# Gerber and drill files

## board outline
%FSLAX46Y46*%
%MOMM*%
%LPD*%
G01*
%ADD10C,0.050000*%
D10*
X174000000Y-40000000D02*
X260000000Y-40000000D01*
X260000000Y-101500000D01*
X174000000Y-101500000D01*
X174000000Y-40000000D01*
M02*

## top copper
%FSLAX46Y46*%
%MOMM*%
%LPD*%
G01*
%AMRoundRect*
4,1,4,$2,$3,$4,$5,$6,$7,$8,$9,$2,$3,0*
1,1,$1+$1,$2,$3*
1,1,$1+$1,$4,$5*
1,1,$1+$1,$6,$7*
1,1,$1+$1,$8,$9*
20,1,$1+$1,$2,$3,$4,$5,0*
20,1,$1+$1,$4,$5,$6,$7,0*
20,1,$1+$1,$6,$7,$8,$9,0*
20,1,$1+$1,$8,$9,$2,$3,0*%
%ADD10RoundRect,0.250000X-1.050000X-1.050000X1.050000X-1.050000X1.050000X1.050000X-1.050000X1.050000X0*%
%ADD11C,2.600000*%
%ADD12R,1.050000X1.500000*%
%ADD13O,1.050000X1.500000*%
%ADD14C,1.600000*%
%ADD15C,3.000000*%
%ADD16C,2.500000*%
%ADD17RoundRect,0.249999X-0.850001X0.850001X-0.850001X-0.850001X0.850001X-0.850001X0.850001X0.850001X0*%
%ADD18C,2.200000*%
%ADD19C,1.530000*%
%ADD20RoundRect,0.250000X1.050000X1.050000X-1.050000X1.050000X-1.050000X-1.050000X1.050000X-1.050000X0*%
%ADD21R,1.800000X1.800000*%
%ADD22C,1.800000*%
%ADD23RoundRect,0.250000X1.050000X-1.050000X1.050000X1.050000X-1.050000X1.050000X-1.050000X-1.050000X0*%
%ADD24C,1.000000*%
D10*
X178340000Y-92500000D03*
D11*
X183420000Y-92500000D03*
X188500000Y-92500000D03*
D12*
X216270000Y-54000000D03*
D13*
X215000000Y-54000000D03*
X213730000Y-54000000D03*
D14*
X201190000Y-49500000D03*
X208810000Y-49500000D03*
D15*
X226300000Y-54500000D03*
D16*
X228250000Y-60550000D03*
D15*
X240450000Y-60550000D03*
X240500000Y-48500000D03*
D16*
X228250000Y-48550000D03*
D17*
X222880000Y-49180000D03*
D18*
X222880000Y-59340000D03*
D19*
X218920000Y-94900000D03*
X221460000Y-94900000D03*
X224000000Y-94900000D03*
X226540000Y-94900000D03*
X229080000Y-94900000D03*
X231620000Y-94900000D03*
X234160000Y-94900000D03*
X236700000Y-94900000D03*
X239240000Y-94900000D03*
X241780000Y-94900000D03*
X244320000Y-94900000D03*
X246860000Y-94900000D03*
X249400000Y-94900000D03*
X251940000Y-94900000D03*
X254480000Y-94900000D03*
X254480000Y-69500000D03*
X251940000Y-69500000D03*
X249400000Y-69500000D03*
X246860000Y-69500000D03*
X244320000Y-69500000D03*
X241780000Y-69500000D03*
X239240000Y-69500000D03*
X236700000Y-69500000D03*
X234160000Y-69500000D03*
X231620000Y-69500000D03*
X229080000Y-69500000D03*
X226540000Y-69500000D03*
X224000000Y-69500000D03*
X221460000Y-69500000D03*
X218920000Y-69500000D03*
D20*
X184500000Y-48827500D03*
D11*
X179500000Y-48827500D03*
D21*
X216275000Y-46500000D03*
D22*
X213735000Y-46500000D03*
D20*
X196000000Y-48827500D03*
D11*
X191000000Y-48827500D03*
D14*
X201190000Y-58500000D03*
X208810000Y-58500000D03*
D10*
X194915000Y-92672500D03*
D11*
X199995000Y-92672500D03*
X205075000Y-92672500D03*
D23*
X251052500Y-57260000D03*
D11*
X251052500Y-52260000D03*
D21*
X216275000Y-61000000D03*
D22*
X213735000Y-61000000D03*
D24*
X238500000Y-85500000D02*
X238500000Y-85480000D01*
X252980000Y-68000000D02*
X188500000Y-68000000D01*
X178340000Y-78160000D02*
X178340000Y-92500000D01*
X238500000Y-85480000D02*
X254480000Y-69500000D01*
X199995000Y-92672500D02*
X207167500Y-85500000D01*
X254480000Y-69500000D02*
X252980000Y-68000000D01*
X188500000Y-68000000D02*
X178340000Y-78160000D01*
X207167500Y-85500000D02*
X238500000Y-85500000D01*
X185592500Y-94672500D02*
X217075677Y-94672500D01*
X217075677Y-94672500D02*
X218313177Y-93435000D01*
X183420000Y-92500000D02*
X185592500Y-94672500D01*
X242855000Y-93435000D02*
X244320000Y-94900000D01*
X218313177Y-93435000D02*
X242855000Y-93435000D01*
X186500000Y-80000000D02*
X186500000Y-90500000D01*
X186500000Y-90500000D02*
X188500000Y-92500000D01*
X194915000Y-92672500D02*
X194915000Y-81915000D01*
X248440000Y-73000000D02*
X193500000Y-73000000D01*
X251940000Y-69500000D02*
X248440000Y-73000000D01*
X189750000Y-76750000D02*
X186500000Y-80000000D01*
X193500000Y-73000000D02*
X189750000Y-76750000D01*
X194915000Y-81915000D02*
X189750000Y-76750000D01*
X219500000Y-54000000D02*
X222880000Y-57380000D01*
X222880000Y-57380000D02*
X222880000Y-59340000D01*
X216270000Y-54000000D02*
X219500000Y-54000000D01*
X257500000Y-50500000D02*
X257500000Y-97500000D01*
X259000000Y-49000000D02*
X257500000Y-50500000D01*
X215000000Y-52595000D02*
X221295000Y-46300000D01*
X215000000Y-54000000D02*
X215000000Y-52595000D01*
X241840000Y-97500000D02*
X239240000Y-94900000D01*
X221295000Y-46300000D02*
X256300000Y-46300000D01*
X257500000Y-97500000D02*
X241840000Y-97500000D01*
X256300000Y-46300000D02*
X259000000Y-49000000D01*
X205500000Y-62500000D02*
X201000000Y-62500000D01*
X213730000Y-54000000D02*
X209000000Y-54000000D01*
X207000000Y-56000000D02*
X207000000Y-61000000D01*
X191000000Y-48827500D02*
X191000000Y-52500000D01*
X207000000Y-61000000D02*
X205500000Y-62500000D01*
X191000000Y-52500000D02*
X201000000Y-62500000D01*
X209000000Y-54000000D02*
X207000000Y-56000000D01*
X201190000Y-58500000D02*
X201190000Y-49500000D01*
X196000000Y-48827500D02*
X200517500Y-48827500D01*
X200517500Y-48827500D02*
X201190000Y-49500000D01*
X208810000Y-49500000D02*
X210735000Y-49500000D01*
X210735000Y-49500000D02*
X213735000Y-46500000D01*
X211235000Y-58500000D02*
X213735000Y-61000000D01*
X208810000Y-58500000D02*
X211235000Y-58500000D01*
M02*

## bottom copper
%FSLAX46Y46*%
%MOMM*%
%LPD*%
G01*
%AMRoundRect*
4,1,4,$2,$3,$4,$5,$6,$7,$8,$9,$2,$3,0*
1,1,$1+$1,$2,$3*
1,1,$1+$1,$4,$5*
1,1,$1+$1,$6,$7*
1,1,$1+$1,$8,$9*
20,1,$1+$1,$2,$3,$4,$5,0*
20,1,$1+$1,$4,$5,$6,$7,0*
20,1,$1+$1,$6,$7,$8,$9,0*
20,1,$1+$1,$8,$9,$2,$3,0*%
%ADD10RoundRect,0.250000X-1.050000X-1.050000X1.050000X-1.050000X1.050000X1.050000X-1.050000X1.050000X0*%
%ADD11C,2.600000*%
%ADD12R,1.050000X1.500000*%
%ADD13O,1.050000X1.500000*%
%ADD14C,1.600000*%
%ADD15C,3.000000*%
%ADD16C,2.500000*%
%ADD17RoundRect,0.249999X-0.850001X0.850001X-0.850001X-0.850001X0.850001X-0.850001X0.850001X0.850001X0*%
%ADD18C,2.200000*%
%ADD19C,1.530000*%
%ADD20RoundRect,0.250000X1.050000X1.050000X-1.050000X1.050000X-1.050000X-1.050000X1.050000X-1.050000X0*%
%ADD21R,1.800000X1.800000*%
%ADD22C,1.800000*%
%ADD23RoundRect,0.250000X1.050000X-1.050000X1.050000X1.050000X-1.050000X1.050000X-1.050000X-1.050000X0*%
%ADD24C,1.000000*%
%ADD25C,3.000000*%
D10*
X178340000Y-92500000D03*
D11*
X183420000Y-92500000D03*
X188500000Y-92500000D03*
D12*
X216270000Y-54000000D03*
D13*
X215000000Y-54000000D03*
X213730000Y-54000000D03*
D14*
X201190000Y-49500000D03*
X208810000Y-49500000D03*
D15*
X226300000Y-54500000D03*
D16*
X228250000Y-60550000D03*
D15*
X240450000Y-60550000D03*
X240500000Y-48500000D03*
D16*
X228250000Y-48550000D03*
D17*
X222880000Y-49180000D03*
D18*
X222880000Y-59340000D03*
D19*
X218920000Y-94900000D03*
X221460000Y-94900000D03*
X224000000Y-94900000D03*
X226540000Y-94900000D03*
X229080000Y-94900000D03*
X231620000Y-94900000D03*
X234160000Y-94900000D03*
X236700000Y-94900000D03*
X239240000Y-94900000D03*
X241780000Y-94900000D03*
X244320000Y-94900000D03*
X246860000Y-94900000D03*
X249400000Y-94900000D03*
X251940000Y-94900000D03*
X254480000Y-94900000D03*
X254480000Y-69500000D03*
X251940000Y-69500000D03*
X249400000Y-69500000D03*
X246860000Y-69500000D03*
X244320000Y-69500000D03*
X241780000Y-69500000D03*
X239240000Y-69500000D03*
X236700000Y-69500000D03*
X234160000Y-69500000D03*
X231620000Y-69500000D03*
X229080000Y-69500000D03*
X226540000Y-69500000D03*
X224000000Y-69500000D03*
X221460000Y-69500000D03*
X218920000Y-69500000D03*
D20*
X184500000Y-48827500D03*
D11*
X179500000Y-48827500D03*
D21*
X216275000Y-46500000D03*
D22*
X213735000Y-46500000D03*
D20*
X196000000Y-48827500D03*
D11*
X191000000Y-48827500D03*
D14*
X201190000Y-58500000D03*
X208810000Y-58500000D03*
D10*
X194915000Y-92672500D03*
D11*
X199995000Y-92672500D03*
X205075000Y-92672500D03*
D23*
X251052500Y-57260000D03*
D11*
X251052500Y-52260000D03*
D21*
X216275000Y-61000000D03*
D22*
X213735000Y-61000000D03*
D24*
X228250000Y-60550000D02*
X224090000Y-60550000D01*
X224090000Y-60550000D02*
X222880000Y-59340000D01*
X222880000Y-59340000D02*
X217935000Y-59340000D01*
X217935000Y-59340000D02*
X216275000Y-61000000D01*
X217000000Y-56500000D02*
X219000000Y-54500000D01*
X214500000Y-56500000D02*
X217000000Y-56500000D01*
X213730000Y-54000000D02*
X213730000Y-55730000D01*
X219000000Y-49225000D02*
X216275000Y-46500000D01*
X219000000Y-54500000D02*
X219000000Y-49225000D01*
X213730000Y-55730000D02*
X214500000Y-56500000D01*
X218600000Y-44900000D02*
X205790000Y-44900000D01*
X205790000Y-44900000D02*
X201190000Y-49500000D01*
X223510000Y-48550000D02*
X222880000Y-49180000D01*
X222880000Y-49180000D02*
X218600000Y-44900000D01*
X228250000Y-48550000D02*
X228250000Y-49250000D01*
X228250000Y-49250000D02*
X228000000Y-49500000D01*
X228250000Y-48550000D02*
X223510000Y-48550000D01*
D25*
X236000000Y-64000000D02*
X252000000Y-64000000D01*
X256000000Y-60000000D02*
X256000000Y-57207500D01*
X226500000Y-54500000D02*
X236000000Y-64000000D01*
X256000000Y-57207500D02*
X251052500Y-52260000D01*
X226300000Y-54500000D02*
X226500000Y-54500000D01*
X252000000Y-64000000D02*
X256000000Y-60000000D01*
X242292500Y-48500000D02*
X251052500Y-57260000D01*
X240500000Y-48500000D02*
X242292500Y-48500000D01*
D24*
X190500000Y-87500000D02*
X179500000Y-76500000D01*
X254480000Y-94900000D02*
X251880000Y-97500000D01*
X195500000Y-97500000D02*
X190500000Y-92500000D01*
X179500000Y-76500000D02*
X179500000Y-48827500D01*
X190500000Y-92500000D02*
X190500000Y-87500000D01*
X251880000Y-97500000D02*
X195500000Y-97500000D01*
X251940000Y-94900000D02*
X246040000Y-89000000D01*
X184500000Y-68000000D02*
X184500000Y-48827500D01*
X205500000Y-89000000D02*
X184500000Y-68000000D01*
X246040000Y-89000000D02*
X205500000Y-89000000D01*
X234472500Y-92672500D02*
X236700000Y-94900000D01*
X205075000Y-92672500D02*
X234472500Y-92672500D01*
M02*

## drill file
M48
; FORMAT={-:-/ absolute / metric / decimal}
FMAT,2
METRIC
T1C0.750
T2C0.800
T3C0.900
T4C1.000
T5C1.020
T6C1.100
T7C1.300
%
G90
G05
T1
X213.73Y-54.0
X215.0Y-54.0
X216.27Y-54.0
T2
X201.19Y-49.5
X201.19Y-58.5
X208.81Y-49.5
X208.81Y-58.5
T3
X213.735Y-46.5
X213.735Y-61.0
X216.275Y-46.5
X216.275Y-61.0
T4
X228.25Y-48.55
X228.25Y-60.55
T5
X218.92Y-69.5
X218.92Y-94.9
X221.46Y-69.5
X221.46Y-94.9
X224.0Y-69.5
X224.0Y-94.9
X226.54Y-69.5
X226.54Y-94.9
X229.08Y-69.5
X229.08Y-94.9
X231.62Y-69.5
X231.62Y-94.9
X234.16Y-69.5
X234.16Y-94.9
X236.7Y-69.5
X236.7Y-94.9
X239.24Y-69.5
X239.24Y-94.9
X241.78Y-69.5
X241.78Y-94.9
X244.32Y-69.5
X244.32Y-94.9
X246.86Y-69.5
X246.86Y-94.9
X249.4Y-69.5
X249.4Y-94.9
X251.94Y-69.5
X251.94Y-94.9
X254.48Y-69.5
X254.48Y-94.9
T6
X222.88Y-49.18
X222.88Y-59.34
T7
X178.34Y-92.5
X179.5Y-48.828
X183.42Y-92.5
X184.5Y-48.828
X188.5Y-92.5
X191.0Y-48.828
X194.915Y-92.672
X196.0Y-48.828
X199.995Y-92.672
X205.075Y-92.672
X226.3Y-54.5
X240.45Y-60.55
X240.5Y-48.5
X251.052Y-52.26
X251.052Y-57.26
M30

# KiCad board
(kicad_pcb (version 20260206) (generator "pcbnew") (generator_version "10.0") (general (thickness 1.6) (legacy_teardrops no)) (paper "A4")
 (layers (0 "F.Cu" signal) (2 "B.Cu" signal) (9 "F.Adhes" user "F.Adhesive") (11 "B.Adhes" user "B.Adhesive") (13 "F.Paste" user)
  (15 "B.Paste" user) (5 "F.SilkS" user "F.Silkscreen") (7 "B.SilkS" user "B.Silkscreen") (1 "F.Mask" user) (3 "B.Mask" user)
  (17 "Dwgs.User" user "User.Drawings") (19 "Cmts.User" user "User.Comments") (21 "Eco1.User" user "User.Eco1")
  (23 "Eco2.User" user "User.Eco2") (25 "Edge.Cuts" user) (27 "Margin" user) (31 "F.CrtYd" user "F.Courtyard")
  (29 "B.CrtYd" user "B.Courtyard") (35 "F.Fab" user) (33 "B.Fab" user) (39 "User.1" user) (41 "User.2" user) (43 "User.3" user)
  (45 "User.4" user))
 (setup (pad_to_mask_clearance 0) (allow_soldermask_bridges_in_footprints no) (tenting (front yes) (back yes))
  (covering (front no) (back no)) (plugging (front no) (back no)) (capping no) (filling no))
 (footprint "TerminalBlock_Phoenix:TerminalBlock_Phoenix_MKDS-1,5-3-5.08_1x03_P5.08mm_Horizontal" (layer "F.Cu") (at 178.34 92.5)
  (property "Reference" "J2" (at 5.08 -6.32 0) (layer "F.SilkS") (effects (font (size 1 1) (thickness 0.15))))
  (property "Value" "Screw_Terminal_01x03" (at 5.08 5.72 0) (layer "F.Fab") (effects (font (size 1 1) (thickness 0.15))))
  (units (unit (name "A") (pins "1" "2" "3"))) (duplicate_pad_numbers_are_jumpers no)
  (pad "1" thru_hole roundrect (at 0 0) (size 2.6 2.6) (drill 1.3) (layers "*.Cu" "*.Mask") (remove_unused_layers no)
   (roundrect_rratio 0.096154) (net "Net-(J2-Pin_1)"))
  (pad "2" thru_hole circle (at 5.08 0) (size 2.6 2.6) (drill 1.3) (layers "*.Cu" "*.Mask") (remove_unused_layers no) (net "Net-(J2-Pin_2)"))
  (pad "3" thru_hole circle (at 10.16 0) (size 2.6 2.6) (drill 1.3) (layers "*.Cu" "*.Mask") (remove_unused_layers no)
   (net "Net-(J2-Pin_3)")))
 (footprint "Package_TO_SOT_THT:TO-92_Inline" (layer "F.Cu") (at 216.27 54 180)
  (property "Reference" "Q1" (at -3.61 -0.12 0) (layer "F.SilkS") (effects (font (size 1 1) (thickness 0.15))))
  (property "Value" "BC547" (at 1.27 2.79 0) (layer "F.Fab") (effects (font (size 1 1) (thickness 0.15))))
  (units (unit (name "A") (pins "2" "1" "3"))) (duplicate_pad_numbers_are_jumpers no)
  (pad "1" thru_hole rect (at 0 0 180) (size 1.05 1.5) (drill 0.75) (layers "*.Cu" "*.Mask") (remove_unused_layers no) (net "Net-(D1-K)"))
  (pad "2" thru_hole oval (at 1.27 0 180) (size 1.05 1.5) (drill 0.75) (layers "*.Cu" "*.Mask") (remove_unused_layers no) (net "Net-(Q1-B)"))
  (pad "3" thru_hole oval (at 2.54 0 180) (size 1.05 1.5) (drill 0.75) (layers "*.Cu" "*.Mask") (remove_unused_layers no) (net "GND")))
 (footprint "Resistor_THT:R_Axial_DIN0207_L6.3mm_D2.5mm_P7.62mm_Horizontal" (layer "F.Cu") (at 201.19 49.5)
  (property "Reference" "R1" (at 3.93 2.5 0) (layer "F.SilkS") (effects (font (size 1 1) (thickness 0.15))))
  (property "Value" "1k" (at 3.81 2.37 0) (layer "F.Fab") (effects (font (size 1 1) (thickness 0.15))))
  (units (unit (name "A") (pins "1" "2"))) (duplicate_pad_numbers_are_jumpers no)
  (pad "1" thru_hole circle (at 0 0) (size 1.6 1.6) (drill 0.8) (layers "*.Cu" "*.Mask") (remove_unused_layers no) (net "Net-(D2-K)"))
  (pad "2" thru_hole circle (at 7.62 0) (size 1.6 1.6) (drill 0.8) (layers "*.Cu" "*.Mask") (remove_unused_layers no) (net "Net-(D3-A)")))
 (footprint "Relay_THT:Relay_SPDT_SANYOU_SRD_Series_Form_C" (layer "F.Cu") (at 226.3 54.5)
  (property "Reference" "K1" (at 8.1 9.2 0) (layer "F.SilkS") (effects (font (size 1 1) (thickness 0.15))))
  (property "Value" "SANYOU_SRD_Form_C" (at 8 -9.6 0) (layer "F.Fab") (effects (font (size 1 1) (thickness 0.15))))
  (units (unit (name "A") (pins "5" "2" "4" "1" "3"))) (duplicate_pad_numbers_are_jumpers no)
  (pad "1" thru_hole circle (at 0 0 90) (size 3 3) (drill 1.3) (layers "*.Cu" "*.Mask") (remove_unused_layers no) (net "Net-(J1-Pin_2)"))
  (pad "2" thru_hole circle (at 1.95 6.05 90) (size 2.5 2.5) (drill 1) (layers "*.Cu" "*.Mask") (remove_unused_layers no) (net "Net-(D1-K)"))
  (pad "3" thru_hole circle (at 14.15 6.05 90) (size 3 3) (drill 1.3) (layers "*.Cu" "*.Mask") (remove_unused_layers no)
   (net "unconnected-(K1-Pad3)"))
  (pad "4" thru_hole circle (at 14.2 -6 90) (size 3 3) (drill 1.3) (layers "*.Cu" "*.Mask") (remove_unused_layers no) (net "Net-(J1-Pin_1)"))
  (pad "5" thru_hole circle (at 1.95 -5.95 90) (size 2.5 2.5) (drill 1) (layers "*.Cu" "*.Mask") (remove_unused_layers no)
   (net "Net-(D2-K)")))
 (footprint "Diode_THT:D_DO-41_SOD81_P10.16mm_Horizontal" (layer "F.Cu") (at 222.88 49.18 -90)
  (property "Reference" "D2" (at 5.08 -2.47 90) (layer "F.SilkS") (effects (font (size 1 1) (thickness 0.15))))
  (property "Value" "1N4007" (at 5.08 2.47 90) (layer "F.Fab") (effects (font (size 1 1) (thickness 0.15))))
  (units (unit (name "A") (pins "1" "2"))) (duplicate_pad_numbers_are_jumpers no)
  (pad "1" thru_hole roundrect (at 0 0 270) (size 2.2 2.2) (drill 1.1) (layers "*.Cu" "*.Mask") (remove_unused_layers no)
   (roundrect_rratio 0.113636) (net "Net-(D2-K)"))
  (pad "2" thru_hole circle (at 10.16 0 270) (size 2.2 2.2) (drill 1.1) (layers "*.Cu" "*.Mask") (remove_unused_layers no)
   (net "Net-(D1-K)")))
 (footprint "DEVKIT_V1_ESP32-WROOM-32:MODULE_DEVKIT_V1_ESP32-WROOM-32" (layer "F.Cu") (at 231.61 82.2 90)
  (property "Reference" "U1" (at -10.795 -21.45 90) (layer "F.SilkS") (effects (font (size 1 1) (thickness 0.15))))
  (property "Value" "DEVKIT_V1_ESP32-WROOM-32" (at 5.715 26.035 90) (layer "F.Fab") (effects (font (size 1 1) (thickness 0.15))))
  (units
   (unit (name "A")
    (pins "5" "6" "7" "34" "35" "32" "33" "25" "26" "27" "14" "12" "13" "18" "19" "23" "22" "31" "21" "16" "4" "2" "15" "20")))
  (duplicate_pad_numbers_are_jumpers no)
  (pad "5" thru_hole circle (at -12.7 -12.69 90) (size 1.53 1.53) (drill 1.02) (layers "*.Cu" "*.Mask") (remove_unused_layers no)
   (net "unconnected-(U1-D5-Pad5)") (solder_mask_margin 0.102))
  (pad "6" thru_hole circle (at -12.7 -10.15 90) (size 1.53 1.53) (drill 1.02) (layers "*.Cu" "*.Mask") (remove_unused_layers no)
   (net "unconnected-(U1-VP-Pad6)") (solder_mask_margin 0.102))
  (pad "7" thru_hole circle (at -12.7 -7.61 90) (size 1.53 1.53) (drill 1.02) (layers "*.Cu" "*.Mask") (remove_unused_layers no)
   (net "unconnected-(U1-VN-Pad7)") (solder_mask_margin 0.102))
  (pad "8" thru_hole circle (at -12.7 -5.07 90) (size 1.53 1.53) (drill 1.02) (layers "*.Cu" "*.Mask") (remove_unused_layers no)
   (solder_mask_margin 0.102))
  (pad "9" thru_hole circle (at -12.7 -2.53 90) (size 1.53 1.53) (drill 1.02) (layers "*.Cu" "*.Mask") (remove_unused_layers no)
   (solder_mask_margin 0.102))
  (pad "10" thru_hole circle (at -12.7 0.01 90) (size 1.53 1.53) (drill 1.02) (layers "*.Cu" "*.Mask") (remove_unused_layers no)
   (solder_mask_margin 0.102))
  (pad "11" thru_hole circle (at -12.7 2.55 90) (size 1.53 1.53) (drill 1.02) (layers "*.Cu" "*.Mask") (remove_unused_layers no)
   (solder_mask_margin 0.102))
  (pad "12" thru_hole circle (at -12.7 5.09 90) (size 1.53 1.53) (drill 1.02) (layers "*.Cu" "*.Mask") (remove_unused_layers no)
   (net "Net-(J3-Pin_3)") (solder_mask_margin 0.102))
  (pad "13" thru_hole circle (at -12.7 7.63 90) (size 1.53 1.53) (drill 1.02) (layers "*.Cu" "*.Mask") (remove_unused_layers no)
   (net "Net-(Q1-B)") (solder_mask_margin 0.102))
  (pad "14" thru_hole circle (at -12.7 10.17 90) (size 1.53 1.53) (drill 1.02) (layers "*.Cu" "*.Mask") (remove_unused_layers no)
   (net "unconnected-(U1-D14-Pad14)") (solder_mask_margin 0.102))
  (pad "15" thru_hole circle (at -12.7 12.71 90) (size 1.53 1.53) (drill 1.02) (layers "*.Cu" "*.Mask") (remove_unused_layers no)
   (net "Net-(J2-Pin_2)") (solder_mask_margin 0.102))
  (pad "16" thru_hole circle (at -12.7 15.25 90) (size 1.53 1.53) (drill 1.02) (layers "*.Cu" "*.Mask") (remove_unused_layers no)
   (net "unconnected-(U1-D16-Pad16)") (solder_mask_margin 0.102))
  (pad "17" thru_hole circle (at -12.7 17.79 90) (size 1.53 1.53) (drill 1.02) (layers "*.Cu" "*.Mask") (remove_unused_layers no)
   (solder_mask_margin 0.102))
  (pad "18" thru_hole circle (at -12.7 20.33 90) (size 1.53 1.53) (drill 1.02) (layers "*.Cu" "*.Mask") (remove_unused_layers no)
   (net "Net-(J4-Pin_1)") (solder_mask_margin 0.102))
  (pad "19" thru_hole circle (at -12.7 22.87 90) (size 1.53 1.53) (drill 1.02) (layers "*.Cu" "*.Mask") (remove_unused_layers no)
   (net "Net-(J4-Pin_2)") (solder_mask_margin 0.102))
  (pad "20" thru_hole circle (at 12.7 22.87 90) (size 1.53 1.53) (drill 1.02) (layers "*.Cu" "*.Mask") (remove_unused_layers no)
   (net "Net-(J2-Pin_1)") (solder_mask_margin 0.102))
  (pad "21" thru_hole circle (at 12.7 20.33 90) (size 1.53 1.53) (drill 1.02) (layers "*.Cu" "*.Mask") (remove_unused_layers no)
   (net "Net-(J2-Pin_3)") (solder_mask_margin 0.102))
  (pad "22" thru_hole circle (at 12.7 17.79 90) (size 1.53 1.53) (drill 1.02) (layers "*.Cu" "*.Mask") (remove_unused_layers no)
   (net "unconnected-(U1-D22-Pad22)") (solder_mask_margin 0.102))
  (pad "23" thru_hole circle (at 12.7 15.25 90) (size 1.53 1.53) (drill 1.02) (layers "*.Cu" "*.Mask") (remove_unused_layers no)
   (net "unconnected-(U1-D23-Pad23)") (solder_mask_margin 0.102))
  (pad "24" thru_hole circle (at 12.7 12.71 90) (size 1.53 1.53) (drill 1.02) (layers "*.Cu" "*.Mask") (remove_unused_layers no)
   (solder_mask_margin 0.102))
  (pad "25" thru_hole circle (at 12.7 10.17 90) (size 1.53 1.53) (drill 1.02) (layers "*.Cu" "*.Mask") (remove_unused_layers no)
   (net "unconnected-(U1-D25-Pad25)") (solder_mask_margin 0.102))
  (pad "26" thru_hole circle (at 12.7 7.63 90) (size 1.53 1.53) (drill 1.02) (layers "*.Cu" "*.Mask") (remove_unused_layers no)
   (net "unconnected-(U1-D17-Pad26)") (solder_mask_margin 0.102))
  (pad "27" thru_hole circle (at 12.7 5.09 90) (size 1.53 1.53) (drill 1.02) (layers "*.Cu" "*.Mask") (remove_unused_layers no)
   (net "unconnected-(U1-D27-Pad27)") (solder_mask_margin 0.102))
  (pad "28" thru_hole circle (at 12.7 2.55 90) (size 1.53 1.53) (drill 1.02) (layers "*.Cu" "*.Mask") (remove_unused_layers no)
   (solder_mask_margin 0.102))
  (pad "29" thru_hole circle (at 12.7 0.01 90) (size 1.53 1.53) (drill 1.02) (layers "*.Cu" "*.Mask") (remove_unused_layers no)
   (solder_mask_margin 0.102))
  (pad "30" thru_hole circle (at 12.7 -2.53 90) (size 1.53 1.53) (drill 1.02) (layers "*.Cu" "*.Mask") (remove_unused_layers no)
   (solder_mask_margin 0.102))
  (pad "31" thru_hole circle (at 12.7 -5.07 90) (size 1.53 1.53) (drill 1.02) (layers "*.Cu" "*.Mask") (remove_unused_layers no)
   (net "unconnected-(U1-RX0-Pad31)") (solder_mask_margin 0.102))
  (pad "32" thru_hole circle (at 12.7 -7.61 90) (size 1.53 1.53) (drill 1.02) (layers "*.Cu" "*.Mask") (remove_unused_layers no)
   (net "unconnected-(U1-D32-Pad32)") (solder_mask_margin 0.102))
  (pad "33" thru_hole circle (at 12.7 -10.15 90) (size 1.53 1.53) (drill 1.02) (layers "*.Cu" "*.Mask") (remove_unused_layers no)
   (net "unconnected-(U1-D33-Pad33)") (solder_mask_margin 0.102))
  (pad "34" thru_hole circle (at 12.7 -12.69 90) (size 1.53 1.53) (drill 1.02) (layers "*.Cu" "*.Mask") (remove_unused_layers no)
   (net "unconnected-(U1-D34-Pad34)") (solder_mask_margin 0.102)))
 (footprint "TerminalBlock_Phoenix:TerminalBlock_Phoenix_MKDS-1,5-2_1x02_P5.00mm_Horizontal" (layer "F.Cu") (at 184.5 48.8275 180)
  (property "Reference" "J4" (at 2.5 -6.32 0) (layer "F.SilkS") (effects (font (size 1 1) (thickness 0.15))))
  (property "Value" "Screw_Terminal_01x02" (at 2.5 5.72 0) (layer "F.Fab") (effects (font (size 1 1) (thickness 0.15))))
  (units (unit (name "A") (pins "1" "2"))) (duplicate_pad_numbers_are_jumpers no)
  (pad "1" thru_hole roundrect (at 0 0 180) (size 2.6 2.6) (drill 1.3) (layers "*.Cu" "*.Mask") (remove_unused_layers no)
   (roundrect_rratio 0.096154) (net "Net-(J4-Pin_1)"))
  (pad "2" thru_hole circle (at 5 0 180) (size 2.6 2.6) (drill 1.3) (layers "*.Cu" "*.Mask") (remove_unused_layers no)
   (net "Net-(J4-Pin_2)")))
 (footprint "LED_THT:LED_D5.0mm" (layer "F.Cu") (at 216.275 46.5 180)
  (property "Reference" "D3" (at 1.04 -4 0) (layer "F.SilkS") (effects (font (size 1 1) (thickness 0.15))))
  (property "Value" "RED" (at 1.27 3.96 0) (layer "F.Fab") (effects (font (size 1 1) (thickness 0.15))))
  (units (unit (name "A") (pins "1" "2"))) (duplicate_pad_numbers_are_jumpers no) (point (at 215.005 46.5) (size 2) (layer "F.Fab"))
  (pad "1" thru_hole rect (at 0 0 180) (size 1.8 1.8) (drill 0.9) (layers "*.Cu" "*.Mask") (remove_unused_layers no) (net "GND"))
  (pad "2" thru_hole circle (at 2.54 0 180) (size 1.8 1.8) (drill 0.9) (layers "*.Cu" "*.Mask") (remove_unused_layers no) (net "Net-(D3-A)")))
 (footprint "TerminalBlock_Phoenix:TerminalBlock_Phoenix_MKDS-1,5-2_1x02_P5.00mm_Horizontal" (layer "F.Cu") (at 196 48.8275 180)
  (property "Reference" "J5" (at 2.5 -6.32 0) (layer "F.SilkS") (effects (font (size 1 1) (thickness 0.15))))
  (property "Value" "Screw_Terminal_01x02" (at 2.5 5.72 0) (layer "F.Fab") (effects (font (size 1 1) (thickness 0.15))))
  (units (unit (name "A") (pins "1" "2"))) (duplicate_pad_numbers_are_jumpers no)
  (pad "1" thru_hole roundrect (at 0 0 180) (size 2.6 2.6) (drill 1.3) (layers "*.Cu" "*.Mask") (remove_unused_layers no)
   (roundrect_rratio 0.096154) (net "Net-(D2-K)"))
  (pad "2" thru_hole circle (at 5 0 180) (size 2.6 2.6) (drill 1.3) (layers "*.Cu" "*.Mask") (remove_unused_layers no) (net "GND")))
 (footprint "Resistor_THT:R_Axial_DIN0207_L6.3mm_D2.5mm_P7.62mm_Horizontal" (layer "F.Cu") (at 201.19 58.5)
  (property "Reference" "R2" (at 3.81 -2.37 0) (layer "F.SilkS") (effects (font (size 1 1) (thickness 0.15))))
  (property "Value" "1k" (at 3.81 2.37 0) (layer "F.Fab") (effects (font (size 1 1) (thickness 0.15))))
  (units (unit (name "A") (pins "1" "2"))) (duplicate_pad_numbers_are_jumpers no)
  (pad "1" thru_hole circle (at 0 0) (size 1.6 1.6) (drill 0.8) (layers "*.Cu" "*.Mask") (remove_unused_layers no) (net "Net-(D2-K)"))
  (pad "2" thru_hole circle (at 7.62 0) (size 1.6 1.6) (drill 0.8) (layers "*.Cu" "*.Mask") (remove_unused_layers no) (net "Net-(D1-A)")))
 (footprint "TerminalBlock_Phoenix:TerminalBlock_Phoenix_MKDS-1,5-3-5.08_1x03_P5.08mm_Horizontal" (layer "F.Cu") (at 194.915 92.6725)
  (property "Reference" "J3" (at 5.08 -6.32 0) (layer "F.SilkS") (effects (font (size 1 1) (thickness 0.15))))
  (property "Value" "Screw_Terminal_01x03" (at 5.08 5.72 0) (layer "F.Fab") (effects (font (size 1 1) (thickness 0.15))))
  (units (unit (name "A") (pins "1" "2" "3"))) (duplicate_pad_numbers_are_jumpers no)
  (pad "1" thru_hole roundrect (at 0 0) (size 2.6 2.6) (drill 1.3) (layers "*.Cu" "*.Mask") (remove_unused_layers no)
   (roundrect_rratio 0.096154) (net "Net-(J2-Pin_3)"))
  (pad "2" thru_hole circle (at 5.08 0) (size 2.6 2.6) (drill 1.3) (layers "*.Cu" "*.Mask") (remove_unused_layers no) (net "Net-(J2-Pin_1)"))
  (pad "3" thru_hole circle (at 10.16 0) (size 2.6 2.6) (drill 1.3) (layers "*.Cu" "*.Mask") (remove_unused_layers no)
   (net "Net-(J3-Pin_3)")))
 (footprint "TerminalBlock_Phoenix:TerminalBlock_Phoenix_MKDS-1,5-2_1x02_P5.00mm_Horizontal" (layer "F.Cu") (at 251.0525 57.26 90)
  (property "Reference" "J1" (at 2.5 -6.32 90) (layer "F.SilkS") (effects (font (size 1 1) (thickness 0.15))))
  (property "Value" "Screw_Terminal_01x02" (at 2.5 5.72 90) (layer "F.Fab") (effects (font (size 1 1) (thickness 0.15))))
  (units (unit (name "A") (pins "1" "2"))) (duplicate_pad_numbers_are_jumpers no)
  (pad "1" thru_hole roundrect (at 0 0 90) (size 2.6 2.6) (drill 1.3) (layers "*.Cu" "*.Mask") (remove_unused_layers no)
   (roundrect_rratio 0.096154) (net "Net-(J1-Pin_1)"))
  (pad "2" thru_hole circle (at 5 0 90) (size 2.6 2.6) (drill 1.3) (layers "*.Cu" "*.Mask") (remove_unused_layers no) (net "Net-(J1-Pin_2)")))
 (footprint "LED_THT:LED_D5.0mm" (layer "F.Cu") (at 216.275 61 180)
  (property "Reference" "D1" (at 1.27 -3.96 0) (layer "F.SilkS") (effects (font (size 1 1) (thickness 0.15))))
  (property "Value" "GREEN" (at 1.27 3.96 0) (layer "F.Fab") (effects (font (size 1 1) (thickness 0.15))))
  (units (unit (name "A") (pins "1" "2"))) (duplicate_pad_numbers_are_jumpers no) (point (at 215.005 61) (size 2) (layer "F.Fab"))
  (pad "1" thru_hole rect (at 0 0 180) (size 1.8 1.8) (drill 0.9) (layers "*.Cu" "*.Mask") (remove_unused_layers no) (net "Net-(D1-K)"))
  (pad "2" thru_hole circle (at 2.54 0 180) (size 1.8 1.8) (drill 0.9) (layers "*.Cu" "*.Mask") (remove_unused_layers no) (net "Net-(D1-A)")))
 (gr_rect (start 174 40) (end 260 101.5) (stroke (width 0.05) (type default)) (fill no) (layer "Edge.Cuts"))
 (segment (start 238.5 85.5) (end 238.5 85.48) (width 1) (layer "F.Cu") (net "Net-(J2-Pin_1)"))
 (segment (start 252.98 68) (end 188.5 68) (width 1) (layer "F.Cu") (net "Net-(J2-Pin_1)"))
 (segment (start 178.34 78.16) (end 178.34 92.5) (width 1) (layer "F.Cu") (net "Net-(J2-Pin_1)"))
 (segment (start 238.5 85.48) (end 254.48 69.5) (width 1) (layer "F.Cu") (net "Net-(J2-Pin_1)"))
 (segment (start 199.995 92.6725) (end 207.1675 85.5) (width 1) (layer "F.Cu") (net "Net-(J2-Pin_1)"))
 (segment (start 254.48 69.5) (end 252.98 68) (width 1) (layer "F.Cu") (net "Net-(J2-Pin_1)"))
 (segment (start 188.5 68) (end 178.34 78.16) (width 1) (layer "F.Cu") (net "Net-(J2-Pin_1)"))
 (segment (start 207.1675 85.5) (end 238.5 85.5) (width 1) (layer "F.Cu") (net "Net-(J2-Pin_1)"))
 (segment (start 185.5925 94.6725) (end 217.075677 94.6725) (width 1) (layer "F.Cu") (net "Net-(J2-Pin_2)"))
 (segment (start 217.075677 94.6725) (end 218.313177 93.435) (width 1) (layer "F.Cu") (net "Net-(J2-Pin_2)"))
 (segment (start 183.42 92.5) (end 185.5925 94.6725) (width 1) (layer "F.Cu") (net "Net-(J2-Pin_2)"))
 (segment (start 242.855 93.435) (end 244.32 94.9) (width 1) (layer "F.Cu") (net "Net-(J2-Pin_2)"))
 (segment (start 218.313177 93.435) (end 242.855 93.435) (width 1) (layer "F.Cu") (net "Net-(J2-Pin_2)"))
 (segment (start 186.5 80) (end 186.5 90.5) (width 1) (layer "F.Cu") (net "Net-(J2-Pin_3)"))
 (segment (start 186.5 90.5) (end 188.5 92.5) (width 1) (layer "F.Cu") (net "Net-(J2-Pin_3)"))
 (segment (start 194.915 92.6725) (end 194.915 81.915) (width 1) (layer "F.Cu") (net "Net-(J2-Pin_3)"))
 (segment (start 248.44 73) (end 193.5 73) (width 1) (layer "F.Cu") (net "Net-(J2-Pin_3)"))
 (segment (start 251.94 69.5) (end 248.44 73) (width 1) (layer "F.Cu") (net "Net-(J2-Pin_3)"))
 (segment (start 189.75 76.75) (end 186.5 80) (width 1) (layer "F.Cu") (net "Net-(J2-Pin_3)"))
 (segment (start 193.5 73) (end 189.75 76.75) (width 1) (layer "F.Cu") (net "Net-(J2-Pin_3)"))
 (segment (start 194.915 81.915) (end 189.75 76.75) (width 1) (layer "F.Cu") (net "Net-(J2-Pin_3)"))
 (segment (start 219.5 54) (end 222.88 57.38) (width 1) (layer "F.Cu") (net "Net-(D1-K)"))
 (segment (start 222.88 57.38) (end 222.88 59.34) (width 1) (layer "F.Cu") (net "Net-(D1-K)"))
 (segment (start 216.27 54) (end 219.5 54) (width 1) (layer "F.Cu") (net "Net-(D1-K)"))
 (segment (start 228.25 60.55) (end 224.09 60.55) (width 1) (layer "B.Cu") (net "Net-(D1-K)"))
 (segment (start 224.09 60.55) (end 222.88 59.34) (width 1) (layer "B.Cu") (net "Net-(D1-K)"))
 (segment (start 222.88 59.34) (end 217.935 59.34) (width 1) (layer "B.Cu") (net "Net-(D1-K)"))
 (segment (start 217.935 59.34) (end 216.275 61) (width 1) (layer "B.Cu") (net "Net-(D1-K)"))
 (segment (start 257.5 50.5) (end 257.5 97.5) (width 1) (layer "F.Cu") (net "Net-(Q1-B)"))
 (segment (start 259 49) (end 257.5 50.5) (width 1) (layer "F.Cu") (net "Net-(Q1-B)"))
 (segment (start 215 52.595) (end 221.295 46.3) (width 1) (layer "F.Cu") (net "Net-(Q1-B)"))
 (segment (start 215 54) (end 215 52.595) (width 1) (layer "F.Cu") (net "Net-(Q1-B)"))
 (segment (start 241.84 97.5) (end 239.24 94.9) (width 1) (layer "F.Cu") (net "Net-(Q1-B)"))
 (segment (start 221.295 46.3) (end 256.3 46.3) (width 1) (layer "F.Cu") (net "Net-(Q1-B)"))
 (segment (start 257.5 97.5) (end 241.84 97.5) (width 1) (layer "F.Cu") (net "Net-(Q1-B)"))
 (segment (start 256.3 46.3) (end 259 49) (width 1) (layer "F.Cu") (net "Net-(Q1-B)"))
 (segment (start 205.5 62.5) (end 201 62.5) (width 1) (layer "F.Cu") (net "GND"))
 (segment (start 213.73 54) (end 209 54) (width 1) (layer "F.Cu") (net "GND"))
 (segment (start 207 56) (end 207 61) (width 1) (layer "F.Cu") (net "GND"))
 (segment (start 191 48.8275) (end 191 52.5) (width 1) (layer "F.Cu") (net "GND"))
 (segment (start 207 61) (end 205.5 62.5) (width 1) (layer "F.Cu") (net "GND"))
 (segment (start 191 52.5) (end 201 62.5) (width 1) (layer "F.Cu") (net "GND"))
 (segment (start 209 54) (end 207 56) (width 1) (layer "F.Cu") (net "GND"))
 (segment (start 217 56.5) (end 219 54.5) (width 1) (layer "B.Cu") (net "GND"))
 (segment (start 214.5 56.5) (end 217 56.5) (width 1) (layer "B.Cu") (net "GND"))
 (segment (start 213.73 54) (end 213.73 55.73) (width 1) (layer "B.Cu") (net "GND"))
 (segment (start 219 49.225) (end 216.275 46.5) (width 1) (layer "B.Cu") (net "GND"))
 (segment (start 219 54.5) (end 219 49.225) (width 1) (layer "B.Cu") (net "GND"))
 (segment (start 213.73 55.73) (end 214.5 56.5) (width 1) (layer "B.Cu") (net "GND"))
 (segment (start 201.19 58.5) (end 201.19 49.5) (width 1) (layer "F.Cu") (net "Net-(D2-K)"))
 (segment (start 196 48.8275) (end 200.5175 48.8275) (width 1) (layer "F.Cu") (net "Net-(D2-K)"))
 (segment (start 200.5175 48.8275) (end 201.19 49.5) (width 1) (layer "F.Cu") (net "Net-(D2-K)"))
 (segment (start 218.6 44.9) (end 205.79 44.9) (width 1) (layer "B.Cu") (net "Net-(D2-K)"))
 (segment (start 205.79 44.9) (end 201.19 49.5) (width 1) (layer "B.Cu") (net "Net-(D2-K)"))
 (segment (start 223.51 48.55) (end 222.88 49.18) (width 1) (layer "B.Cu") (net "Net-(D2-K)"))
 (segment (start 222.88 49.18) (end 218.6 44.9) (width 1) (layer "B.Cu") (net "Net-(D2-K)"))
 (segment (start 228.25 48.55) (end 228.25 49.25) (width 1) (layer "B.Cu") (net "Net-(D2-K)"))
 (segment (start 228.25 49.25) (end 228 49.5) (width 1) (layer "B.Cu") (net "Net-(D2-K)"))
 (segment (start 228.25 48.55) (end 223.51 48.55) (width 1) (layer "B.Cu") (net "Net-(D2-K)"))
 (segment (start 208.81 49.5) (end 210.735 49.5) (width 1) (layer "F.Cu") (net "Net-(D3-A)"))
 (segment (start 210.735 49.5) (end 213.735 46.5) (width 1) (layer "F.Cu") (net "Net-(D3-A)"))
 (segment (start 236 64) (end 252 64) (width 3) (layer "B.Cu") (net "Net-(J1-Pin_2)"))
 (segment (start 256 60) (end 256 57.2075) (width 3) (layer "B.Cu") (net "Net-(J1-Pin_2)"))
 (segment (start 226.5 54.5) (end 236 64) (width 3) (layer "B.Cu") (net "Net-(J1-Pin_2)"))
 (segment (start 256 57.2075) (end 251.0525 52.26) (width 3) (layer "B.Cu") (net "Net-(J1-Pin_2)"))
 (segment (start 226.3 54.5) (end 226.5 54.5) (width 3) (layer "B.Cu") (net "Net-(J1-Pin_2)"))
 (segment (start 252 64) (end 256 60) (width 3) (layer "B.Cu") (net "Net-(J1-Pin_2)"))
 (segment (start 242.2925 48.5) (end 251.0525 57.26) (width 3) (layer "B.Cu") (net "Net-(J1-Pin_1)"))
 (segment (start 240.5 48.5) (end 242.2925 48.5) (width 3) (layer "B.Cu") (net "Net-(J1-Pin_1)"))
 (segment (start 211.235 58.5) (end 213.735 61) (width 1) (layer "F.Cu") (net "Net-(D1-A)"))
 (segment (start 208.81 58.5) (end 211.235 58.5) (width 1) (layer "F.Cu") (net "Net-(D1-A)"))
 (segment (start 190.5 87.5) (end 179.5 76.5) (width 1) (layer "B.Cu") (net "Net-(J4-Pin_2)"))
 (segment (start 254.48 94.9) (end 251.88 97.5) (width 1) (layer "B.Cu") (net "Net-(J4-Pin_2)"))
 (segment (start 195.5 97.5) (end 190.5 92.5) (width 1) (layer "B.Cu") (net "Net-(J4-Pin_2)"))
 (segment (start 179.5 76.5) (end 179.5 48.8275) (width 1) (layer "B.Cu") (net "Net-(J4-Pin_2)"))
 (segment (start 190.5 92.5) (end 190.5 87.5) (width 1) (layer "B.Cu") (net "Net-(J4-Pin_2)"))
 (segment (start 251.88 97.5) (end 195.5 97.5) (width 1) (layer "B.Cu") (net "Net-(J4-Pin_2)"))
 (segment (start 251.94 94.9) (end 246.04 89) (width 1) (layer "B.Cu") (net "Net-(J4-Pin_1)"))
 (segment (start 184.5 68) (end 184.5 48.8275) (width 1) (layer "B.Cu") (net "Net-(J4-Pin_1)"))
 (segment (start 205.5 89) (end 184.5 68) (width 1) (layer "B.Cu") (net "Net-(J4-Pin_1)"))
 (segment (start 246.04 89) (end 205.5 89) (width 1) (layer "B.Cu") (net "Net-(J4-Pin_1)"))
 (segment (start 234.4725 92.6725) (end 236.7 94.9) (width 1) (layer "B.Cu") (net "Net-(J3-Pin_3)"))
 (segment (start 205.075 92.6725) (end 234.4725 92.6725) (width 1) (layer "B.Cu") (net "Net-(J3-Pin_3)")))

